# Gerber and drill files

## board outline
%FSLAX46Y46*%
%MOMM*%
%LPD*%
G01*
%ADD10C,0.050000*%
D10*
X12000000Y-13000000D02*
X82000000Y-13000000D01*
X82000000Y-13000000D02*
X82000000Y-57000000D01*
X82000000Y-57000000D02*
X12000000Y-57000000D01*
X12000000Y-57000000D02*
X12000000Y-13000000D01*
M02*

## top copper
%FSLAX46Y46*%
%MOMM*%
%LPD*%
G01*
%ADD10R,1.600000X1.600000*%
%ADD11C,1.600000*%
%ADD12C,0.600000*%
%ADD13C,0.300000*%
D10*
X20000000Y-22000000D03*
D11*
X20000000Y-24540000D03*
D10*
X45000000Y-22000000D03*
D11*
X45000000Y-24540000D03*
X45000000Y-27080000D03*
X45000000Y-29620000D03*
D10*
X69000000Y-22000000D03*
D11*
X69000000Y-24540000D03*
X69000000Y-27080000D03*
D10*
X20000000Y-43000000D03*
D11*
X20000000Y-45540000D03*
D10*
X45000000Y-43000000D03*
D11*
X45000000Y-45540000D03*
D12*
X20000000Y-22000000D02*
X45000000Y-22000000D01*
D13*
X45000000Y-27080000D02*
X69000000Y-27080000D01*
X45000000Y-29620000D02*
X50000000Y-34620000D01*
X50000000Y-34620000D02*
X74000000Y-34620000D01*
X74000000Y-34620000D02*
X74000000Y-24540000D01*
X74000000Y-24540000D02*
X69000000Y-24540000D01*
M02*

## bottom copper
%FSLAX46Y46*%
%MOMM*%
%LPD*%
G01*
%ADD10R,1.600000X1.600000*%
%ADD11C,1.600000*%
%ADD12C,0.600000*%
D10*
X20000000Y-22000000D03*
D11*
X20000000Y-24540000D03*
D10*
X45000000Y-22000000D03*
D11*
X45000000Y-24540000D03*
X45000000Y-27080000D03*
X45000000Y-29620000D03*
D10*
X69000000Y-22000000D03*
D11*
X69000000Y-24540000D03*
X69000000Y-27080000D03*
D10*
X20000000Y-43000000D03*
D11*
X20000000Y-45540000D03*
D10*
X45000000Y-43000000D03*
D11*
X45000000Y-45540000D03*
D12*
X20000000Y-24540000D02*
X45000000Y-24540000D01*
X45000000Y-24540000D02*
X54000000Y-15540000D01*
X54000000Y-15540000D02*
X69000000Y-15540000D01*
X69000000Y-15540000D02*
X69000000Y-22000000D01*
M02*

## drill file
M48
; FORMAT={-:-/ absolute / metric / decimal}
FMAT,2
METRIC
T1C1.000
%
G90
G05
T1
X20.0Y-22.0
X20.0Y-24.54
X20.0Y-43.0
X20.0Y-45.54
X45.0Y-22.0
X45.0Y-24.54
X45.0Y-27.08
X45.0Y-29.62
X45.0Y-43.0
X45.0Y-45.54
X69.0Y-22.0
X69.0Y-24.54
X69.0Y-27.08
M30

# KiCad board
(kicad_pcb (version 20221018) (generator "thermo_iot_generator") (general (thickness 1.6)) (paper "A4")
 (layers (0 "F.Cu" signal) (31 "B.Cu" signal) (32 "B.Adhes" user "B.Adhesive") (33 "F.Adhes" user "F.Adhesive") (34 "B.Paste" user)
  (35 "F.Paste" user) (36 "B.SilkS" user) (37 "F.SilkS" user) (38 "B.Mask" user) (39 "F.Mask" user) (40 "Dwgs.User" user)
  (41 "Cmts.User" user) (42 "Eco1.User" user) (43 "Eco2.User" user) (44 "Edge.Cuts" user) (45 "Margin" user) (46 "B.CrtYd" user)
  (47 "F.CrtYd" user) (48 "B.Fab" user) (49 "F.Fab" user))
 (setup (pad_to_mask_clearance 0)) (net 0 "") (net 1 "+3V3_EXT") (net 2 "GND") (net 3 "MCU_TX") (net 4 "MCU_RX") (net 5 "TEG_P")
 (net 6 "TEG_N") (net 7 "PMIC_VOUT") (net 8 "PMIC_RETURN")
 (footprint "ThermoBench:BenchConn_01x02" (layer "F.Cu") (at 20 22)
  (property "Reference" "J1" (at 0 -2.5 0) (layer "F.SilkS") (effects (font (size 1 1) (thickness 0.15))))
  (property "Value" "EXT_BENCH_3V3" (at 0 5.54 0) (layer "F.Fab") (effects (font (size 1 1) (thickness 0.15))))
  (pad "1" thru_hole rect (at 0 0) (size 1.6 1.6) (drill 1.0) (layers "*.Cu" "*.Mask") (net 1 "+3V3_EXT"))
  (pad "2" thru_hole circle (at 0 2.54) (size 1.6 1.6) (drill 1.0) (layers "*.Cu" "*.Mask") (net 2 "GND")))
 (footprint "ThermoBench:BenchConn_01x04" (layer "F.Cu") (at 45 22)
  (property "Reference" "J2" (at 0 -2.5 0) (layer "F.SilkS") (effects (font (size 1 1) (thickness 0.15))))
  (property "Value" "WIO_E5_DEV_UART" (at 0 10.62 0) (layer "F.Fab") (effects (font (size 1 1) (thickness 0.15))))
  (pad "1" thru_hole rect (at 0 0) (size 1.6 1.6) (drill 1.0) (layers "*.Cu" "*.Mask") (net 1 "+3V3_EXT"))
  (pad "2" thru_hole circle (at 0 2.54) (size 1.6 1.6) (drill 1.0) (layers "*.Cu" "*.Mask") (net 2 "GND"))
  (pad "3" thru_hole circle (at 0 5.08) (size 1.6 1.6) (drill 1.0) (layers "*.Cu" "*.Mask") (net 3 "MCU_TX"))
  (pad "4" thru_hole circle (at 0 7.62) (size 1.6 1.6) (drill 1.0) (layers "*.Cu" "*.Mask") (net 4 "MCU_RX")))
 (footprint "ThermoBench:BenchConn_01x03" (layer "F.Cu") (at 69 22)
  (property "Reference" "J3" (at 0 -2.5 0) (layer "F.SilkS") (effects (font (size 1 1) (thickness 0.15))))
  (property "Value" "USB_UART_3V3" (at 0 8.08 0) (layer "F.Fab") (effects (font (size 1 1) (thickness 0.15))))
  (pad "1" thru_hole rect (at 0 0) (size 1.6 1.6) (drill 1.0) (layers "*.Cu" "*.Mask") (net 2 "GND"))
  (pad "2" thru_hole circle (at 0 2.54) (size 1.6 1.6) (drill 1.0) (layers "*.Cu" "*.Mask") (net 4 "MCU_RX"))
  (pad "3" thru_hole circle (at 0 5.08) (size 1.6 1.6) (drill 1.0) (layers "*.Cu" "*.Mask") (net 3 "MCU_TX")))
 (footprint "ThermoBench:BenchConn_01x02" (layer "F.Cu") (at 20 43)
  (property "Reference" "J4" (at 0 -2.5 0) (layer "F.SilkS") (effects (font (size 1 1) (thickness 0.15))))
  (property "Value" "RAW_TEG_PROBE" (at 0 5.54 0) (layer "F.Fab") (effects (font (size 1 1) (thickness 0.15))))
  (pad "1" thru_hole rect (at 0 0) (size 1.6 1.6) (drill 1.0) (layers "*.Cu" "*.Mask") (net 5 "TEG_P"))
  (pad "2" thru_hole circle (at 0 2.54) (size 1.6 1.6) (drill 1.0) (layers "*.Cu" "*.Mask") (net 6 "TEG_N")))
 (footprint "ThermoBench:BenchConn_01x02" (layer "F.Cu") (at 45 43)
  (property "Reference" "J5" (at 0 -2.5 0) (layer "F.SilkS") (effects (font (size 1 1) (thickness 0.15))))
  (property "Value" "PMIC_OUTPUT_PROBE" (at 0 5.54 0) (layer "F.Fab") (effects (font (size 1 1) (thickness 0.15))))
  (pad "1" thru_hole rect (at 0 0) (size 1.6 1.6) (drill 1.0) (layers "*.Cu" "*.Mask") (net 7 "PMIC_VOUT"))
  (pad "2" thru_hole circle (at 0 2.54) (size 1.6 1.6) (drill 1.0) (layers "*.Cu" "*.Mask") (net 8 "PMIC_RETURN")))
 (segment (start 20 22) (end 45 22) (width 0.6) (layer "F.Cu") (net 1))
 (segment (start 20 24.54) (end 45 24.54) (width 0.6) (layer "B.Cu") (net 2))
 (segment (start 45 24.54) (end 54 15.54) (width 0.6) (layer "B.Cu") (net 2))
 (segment (start 54 15.54) (end 69 15.54) (width 0.6) (layer "B.Cu") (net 2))
 (segment (start 69 15.54) (end 69 22) (width 0.6) (layer "B.Cu") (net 2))
 (segment (start 45 27.08) (end 69 27.08) (width 0.3) (layer "F.Cu") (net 3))
 (segment (start 45 29.62) (end 50 34.62) (width 0.3) (layer "F.Cu") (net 4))
 (segment (start 50 34.62) (end 74 34.62) (width 0.3) (layer "F.Cu") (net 4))
 (segment (start 74 34.62) (end 74 24.54) (width 0.3) (layer "F.Cu") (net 4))
 (segment (start 74 24.54) (end 69 24.54) (width 0.3) (layer "F.Cu") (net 4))
 (gr_line (start 12 13) (end 82 13) (stroke (width 0.05) (type default)) (layer "Edge.Cuts"))
 (gr_line (start 82 13) (end 82 57) (stroke (width 0.05) (type default)) (layer "Edge.Cuts"))
 (gr_line (start 82 57) (end 12 57) (stroke (width 0.05) (type default)) (layer "Edge.Cuts"))
 (gr_line (start 12 57) (end 12 13) (stroke (width 0.05) (type default)) (layer "Edge.Cuts")))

